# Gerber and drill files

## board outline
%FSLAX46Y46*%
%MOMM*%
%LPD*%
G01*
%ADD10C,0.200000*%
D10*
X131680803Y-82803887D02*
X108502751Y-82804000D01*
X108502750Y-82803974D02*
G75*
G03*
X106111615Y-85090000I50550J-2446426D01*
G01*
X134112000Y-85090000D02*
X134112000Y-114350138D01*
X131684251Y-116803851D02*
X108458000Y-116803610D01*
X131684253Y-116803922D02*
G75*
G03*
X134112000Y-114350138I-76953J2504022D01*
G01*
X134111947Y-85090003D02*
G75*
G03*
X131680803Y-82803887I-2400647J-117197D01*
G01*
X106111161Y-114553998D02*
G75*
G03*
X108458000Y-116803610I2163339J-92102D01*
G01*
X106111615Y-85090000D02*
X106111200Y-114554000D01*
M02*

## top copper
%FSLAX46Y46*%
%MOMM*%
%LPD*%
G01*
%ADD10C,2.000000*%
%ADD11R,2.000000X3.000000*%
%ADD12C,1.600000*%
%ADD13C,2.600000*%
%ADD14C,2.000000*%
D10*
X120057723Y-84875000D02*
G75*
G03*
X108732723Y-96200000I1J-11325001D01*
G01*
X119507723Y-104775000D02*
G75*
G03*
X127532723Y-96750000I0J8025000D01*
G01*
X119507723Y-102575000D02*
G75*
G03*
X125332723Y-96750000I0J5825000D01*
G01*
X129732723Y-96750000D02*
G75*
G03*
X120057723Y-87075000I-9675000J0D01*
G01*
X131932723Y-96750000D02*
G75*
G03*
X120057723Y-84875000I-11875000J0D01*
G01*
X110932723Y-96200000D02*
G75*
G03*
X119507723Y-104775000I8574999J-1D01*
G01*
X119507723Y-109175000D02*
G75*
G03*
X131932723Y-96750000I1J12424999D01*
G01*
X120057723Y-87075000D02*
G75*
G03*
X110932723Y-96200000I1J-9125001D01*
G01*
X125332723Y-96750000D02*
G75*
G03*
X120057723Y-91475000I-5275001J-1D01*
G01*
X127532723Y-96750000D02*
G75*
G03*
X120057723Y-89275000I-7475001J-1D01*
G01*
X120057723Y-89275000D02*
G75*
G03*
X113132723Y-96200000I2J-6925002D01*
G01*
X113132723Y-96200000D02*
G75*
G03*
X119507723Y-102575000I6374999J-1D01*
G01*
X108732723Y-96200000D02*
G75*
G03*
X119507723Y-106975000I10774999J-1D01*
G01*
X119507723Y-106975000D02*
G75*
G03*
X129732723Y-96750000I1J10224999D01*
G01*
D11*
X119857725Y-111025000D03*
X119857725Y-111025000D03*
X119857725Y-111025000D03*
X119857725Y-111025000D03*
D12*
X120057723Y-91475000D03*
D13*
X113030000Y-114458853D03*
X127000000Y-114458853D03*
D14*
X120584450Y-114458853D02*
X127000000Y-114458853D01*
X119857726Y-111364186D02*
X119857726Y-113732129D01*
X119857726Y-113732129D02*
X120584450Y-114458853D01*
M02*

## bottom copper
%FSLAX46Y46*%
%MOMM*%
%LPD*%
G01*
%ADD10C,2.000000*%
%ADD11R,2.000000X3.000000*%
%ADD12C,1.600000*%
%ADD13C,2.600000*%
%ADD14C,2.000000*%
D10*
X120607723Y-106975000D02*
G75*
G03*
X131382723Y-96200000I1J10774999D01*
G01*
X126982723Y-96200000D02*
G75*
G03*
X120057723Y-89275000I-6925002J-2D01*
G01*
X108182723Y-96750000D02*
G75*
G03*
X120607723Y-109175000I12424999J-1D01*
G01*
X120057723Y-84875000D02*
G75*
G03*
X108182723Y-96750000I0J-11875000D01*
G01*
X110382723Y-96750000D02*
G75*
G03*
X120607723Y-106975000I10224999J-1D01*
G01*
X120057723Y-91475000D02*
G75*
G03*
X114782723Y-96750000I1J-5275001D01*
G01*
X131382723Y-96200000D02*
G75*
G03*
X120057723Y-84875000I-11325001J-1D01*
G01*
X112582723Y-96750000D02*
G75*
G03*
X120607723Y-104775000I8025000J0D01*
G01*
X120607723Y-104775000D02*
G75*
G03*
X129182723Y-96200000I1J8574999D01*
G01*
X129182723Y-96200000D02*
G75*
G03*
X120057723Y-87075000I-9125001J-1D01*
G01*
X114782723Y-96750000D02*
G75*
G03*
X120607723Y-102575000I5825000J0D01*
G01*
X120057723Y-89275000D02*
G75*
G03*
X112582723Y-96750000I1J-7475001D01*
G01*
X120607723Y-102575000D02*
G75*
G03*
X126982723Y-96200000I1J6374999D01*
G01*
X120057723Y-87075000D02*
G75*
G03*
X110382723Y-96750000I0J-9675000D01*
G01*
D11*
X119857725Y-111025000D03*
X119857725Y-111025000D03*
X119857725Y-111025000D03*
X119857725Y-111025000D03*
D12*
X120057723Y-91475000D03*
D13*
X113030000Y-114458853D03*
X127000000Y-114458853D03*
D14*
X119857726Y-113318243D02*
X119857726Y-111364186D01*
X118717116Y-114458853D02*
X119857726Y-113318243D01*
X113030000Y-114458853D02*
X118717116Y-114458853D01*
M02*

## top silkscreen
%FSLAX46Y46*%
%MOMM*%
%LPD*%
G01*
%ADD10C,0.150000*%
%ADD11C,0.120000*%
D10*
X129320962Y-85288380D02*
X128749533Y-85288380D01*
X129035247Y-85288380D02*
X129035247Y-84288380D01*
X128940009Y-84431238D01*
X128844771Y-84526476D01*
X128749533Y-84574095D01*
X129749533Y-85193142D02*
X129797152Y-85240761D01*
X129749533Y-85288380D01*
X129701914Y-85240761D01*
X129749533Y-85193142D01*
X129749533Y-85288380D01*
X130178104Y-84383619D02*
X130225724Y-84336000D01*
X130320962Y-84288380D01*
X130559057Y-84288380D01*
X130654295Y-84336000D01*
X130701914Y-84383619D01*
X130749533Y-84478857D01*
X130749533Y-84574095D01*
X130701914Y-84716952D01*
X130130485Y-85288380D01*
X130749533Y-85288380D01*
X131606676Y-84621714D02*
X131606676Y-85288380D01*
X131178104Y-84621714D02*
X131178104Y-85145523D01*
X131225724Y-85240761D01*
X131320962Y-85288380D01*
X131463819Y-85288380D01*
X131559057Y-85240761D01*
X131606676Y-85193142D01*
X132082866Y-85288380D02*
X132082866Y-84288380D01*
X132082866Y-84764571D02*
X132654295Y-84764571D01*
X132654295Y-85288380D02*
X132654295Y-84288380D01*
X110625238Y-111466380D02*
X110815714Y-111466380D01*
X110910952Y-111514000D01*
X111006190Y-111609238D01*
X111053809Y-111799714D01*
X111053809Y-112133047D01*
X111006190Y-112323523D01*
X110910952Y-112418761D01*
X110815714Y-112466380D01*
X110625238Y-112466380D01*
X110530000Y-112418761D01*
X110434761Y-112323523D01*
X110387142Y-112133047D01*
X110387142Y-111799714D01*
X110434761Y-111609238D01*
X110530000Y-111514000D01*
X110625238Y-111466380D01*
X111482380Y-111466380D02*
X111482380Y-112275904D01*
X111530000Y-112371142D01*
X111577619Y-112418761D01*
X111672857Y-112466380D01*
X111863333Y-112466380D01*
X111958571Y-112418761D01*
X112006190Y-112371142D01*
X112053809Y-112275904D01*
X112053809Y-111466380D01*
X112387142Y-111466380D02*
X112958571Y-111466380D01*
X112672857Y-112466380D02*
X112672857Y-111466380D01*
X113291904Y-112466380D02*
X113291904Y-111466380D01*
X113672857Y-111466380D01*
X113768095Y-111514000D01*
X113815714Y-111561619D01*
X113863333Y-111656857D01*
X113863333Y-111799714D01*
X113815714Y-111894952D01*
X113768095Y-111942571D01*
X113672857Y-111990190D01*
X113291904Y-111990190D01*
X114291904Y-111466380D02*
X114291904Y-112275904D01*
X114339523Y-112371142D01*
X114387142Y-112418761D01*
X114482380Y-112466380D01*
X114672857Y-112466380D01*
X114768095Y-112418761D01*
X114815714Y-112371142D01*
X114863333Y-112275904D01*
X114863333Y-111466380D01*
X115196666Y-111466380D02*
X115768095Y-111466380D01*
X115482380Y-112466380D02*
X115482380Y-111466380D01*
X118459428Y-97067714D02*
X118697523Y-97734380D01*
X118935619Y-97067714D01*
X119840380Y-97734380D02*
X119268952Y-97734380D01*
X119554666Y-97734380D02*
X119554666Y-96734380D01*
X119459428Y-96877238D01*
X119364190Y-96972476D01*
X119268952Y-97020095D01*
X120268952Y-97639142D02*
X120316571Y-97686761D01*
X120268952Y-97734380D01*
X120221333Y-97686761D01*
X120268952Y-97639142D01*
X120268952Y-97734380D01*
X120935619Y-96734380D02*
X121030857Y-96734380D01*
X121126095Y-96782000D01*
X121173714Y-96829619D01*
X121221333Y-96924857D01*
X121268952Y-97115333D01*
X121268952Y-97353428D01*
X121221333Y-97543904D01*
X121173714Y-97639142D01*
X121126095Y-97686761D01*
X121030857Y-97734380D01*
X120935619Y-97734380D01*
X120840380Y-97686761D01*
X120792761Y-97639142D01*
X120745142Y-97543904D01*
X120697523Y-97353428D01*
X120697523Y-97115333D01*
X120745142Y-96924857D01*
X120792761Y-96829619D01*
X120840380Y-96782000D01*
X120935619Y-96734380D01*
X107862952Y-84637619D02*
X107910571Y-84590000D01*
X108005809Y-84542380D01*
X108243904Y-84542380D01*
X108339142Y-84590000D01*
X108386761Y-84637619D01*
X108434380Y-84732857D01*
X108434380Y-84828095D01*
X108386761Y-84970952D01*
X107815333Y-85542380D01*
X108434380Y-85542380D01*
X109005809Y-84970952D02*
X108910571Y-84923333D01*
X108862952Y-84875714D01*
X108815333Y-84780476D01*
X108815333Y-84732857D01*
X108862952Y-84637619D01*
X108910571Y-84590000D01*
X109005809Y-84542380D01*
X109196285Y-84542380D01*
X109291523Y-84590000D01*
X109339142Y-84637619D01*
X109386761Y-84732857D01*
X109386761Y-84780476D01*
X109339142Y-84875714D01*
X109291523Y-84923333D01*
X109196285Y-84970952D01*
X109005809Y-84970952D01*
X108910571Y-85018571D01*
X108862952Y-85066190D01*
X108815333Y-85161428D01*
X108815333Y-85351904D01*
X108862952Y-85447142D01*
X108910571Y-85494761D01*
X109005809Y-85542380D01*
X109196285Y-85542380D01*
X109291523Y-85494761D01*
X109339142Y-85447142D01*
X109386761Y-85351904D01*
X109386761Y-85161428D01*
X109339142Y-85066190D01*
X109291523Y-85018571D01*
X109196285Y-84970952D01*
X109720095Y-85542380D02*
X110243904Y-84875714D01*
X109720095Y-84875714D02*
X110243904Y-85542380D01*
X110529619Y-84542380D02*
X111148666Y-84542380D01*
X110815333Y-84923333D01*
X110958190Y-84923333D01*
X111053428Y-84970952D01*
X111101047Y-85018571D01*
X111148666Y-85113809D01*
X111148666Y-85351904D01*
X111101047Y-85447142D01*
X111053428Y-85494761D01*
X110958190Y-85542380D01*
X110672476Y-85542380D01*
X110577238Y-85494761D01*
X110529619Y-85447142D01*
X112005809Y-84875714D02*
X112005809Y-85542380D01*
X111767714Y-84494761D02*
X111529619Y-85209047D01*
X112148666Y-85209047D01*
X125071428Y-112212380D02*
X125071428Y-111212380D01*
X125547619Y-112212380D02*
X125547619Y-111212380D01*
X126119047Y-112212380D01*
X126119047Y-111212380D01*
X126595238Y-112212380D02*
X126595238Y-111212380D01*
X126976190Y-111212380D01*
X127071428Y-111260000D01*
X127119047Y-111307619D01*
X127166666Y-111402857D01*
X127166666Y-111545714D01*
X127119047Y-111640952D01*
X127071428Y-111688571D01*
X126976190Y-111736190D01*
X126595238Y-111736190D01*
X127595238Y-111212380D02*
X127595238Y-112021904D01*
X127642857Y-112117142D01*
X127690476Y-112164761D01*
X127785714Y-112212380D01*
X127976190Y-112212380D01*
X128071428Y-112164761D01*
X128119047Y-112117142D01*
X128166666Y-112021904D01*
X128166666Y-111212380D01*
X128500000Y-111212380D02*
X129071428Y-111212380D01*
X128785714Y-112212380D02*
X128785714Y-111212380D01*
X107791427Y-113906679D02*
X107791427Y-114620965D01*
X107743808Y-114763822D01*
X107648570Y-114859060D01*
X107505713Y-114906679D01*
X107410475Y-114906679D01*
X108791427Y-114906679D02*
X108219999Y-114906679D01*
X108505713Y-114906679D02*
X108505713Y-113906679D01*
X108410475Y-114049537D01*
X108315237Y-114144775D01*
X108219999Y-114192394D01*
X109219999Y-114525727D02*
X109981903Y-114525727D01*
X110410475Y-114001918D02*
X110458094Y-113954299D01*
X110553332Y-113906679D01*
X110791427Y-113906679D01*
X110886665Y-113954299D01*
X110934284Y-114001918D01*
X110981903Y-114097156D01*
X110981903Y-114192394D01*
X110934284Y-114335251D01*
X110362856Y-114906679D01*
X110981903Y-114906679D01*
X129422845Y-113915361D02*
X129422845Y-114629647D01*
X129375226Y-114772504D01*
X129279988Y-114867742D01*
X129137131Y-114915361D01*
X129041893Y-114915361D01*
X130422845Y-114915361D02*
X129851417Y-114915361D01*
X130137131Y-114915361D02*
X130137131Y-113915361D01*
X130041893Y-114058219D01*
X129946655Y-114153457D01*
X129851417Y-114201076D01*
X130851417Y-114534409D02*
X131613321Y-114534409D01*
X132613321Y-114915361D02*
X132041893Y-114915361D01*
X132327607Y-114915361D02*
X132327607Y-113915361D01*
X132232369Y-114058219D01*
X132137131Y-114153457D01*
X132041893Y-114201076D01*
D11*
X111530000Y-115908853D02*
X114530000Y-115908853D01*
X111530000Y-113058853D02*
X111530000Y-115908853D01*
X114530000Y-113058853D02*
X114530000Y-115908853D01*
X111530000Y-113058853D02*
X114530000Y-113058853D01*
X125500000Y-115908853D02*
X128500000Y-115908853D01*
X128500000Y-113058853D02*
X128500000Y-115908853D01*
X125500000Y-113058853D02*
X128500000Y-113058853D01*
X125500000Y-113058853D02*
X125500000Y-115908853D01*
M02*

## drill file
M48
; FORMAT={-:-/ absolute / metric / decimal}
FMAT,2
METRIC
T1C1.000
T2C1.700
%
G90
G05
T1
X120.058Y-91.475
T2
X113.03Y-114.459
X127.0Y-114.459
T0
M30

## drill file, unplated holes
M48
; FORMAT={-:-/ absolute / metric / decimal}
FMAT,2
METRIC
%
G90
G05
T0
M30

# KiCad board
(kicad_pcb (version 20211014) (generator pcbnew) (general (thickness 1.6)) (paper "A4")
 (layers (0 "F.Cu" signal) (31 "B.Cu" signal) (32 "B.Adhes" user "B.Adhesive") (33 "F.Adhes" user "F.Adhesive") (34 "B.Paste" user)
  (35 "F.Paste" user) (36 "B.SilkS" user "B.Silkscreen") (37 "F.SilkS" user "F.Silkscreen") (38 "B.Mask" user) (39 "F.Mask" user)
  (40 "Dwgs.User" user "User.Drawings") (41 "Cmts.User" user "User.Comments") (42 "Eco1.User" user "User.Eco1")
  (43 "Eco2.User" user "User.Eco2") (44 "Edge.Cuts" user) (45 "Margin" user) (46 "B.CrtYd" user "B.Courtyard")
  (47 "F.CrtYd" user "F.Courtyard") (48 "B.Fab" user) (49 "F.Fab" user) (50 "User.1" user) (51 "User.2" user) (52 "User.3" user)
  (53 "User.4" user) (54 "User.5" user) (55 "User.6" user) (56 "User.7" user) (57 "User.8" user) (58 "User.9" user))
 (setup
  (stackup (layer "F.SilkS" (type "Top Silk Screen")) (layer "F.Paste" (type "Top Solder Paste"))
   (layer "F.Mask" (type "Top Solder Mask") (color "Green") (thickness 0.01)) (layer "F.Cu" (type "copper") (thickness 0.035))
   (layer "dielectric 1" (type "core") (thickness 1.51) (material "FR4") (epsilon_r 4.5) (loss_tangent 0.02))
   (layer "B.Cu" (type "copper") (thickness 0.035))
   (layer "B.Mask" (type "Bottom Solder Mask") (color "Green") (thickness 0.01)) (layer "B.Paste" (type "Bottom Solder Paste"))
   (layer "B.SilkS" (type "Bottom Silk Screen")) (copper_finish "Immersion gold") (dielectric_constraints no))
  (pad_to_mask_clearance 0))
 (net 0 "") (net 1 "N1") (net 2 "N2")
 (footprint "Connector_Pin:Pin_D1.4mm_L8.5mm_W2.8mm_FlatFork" (layer "F.Cu") (at 113.03 114.458853)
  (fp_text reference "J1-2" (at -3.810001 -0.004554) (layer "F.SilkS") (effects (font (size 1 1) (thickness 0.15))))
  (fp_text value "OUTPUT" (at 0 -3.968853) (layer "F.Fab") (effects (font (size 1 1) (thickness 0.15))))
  (fp_line (start -1.5 1.45) (end 1.5 1.45) (layer "F.SilkS") (width 0.12))
  (fp_line (start -1.5 -1.4) (end -1.5 1.45) (layer "F.SilkS") (width 0.12))
  (fp_line (start 1.5 -1.4) (end 1.5 1.45) (layer "F.SilkS") (width 0.12))
  (fp_line (start -1.5 -1.4) (end 1.5 -1.4) (layer "F.SilkS") (width 0.12))
  (pad "1" thru_hole circle locked (at 0 0) (size 2.6 2.6) (drill 1.7) (layers *.Cu *.Mask) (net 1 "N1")))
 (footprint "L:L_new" (layer "F.Cu") (at 120.057723 98.2 90) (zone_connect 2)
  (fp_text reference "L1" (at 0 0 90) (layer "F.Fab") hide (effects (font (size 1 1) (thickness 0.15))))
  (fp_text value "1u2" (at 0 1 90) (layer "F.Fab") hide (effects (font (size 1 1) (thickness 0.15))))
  (fp_arc (start 1.45 7.475) (mid -4.224532 5.124532) (end -6.575 -0.55) (layer "F.Cu") (width 2))
  (fp_arc (start -4.375 -0.55) (mid -2.507806 -5.057806) (end 2 -6.925) (layer "F.Cu") (width 2))
  (fp_arc (start 2 -6.925) (mid 6.896714 -4.896714) (end 8.925 0) (layer "F.Cu") (width 2))
  (fp_arc (start 1.45 11.875) (mid -7.335802 8.235802) (end -10.975 -0.55) (layer "F.Cu") (width 2))
  (fp_arc (start 1.45 9.675) (mid -5.780167 6.680167) (end -8.775 -0.55) (layer "F.Cu") (width 2))
  (fp_arc (start -8.775 -0.55) (mid -5.619076 -8.169076) (end 2 -11.325) (layer "F.Cu") (width 2))
  (fp_arc (start 8.925 0) (mid 6.735623 5.285623) (end 1.45 7.475) (layer "F.Cu") (width 2))
  (fp_arc (start 13.325 0) (mid 9.846893 8.396893) (end 1.45 11.875) (layer "F.Cu") (width 2))
  (fp_arc (start 11.125 0) (mid 8.291258 6.841258) (end 1.45 9.675) (layer "F.Cu") (width 2))
  (fp_arc (start 2 -11.325) (mid 10.007984 -8.007984) (end 13.325 0) (layer "F.Cu") (width 2))
  (fp_arc (start 1.45 5.275) (mid -2.668897 3.568897) (end -4.375 -0.55) (layer "F.Cu") (width 2))
  (fp_arc (start 2 -9.125) (mid 8.452349 -6.452349) (end 11.125 0) (layer "F.Cu") (width 2))
  (fp_arc (start -6.575 -0.55) (mid -4.063441 -6.613441) (end 2 -9.125) (layer "F.Cu") (width 2))
  (fp_arc (start 6.725 0) (mid 5.179988 3.729988) (end 1.45 5.275) (layer "F.Cu") (width 2))
  (fp_arc (start -8.775 0.55) (mid -5.780167 -6.680167) (end 1.45 -9.675) (layer "B.Cu") (width 2))
  (fp_arc (start 2 11.325) (mid -5.619076 8.169076) (end -8.775 0.55) (layer "B.Cu") (width 2))
  (fp_arc (start 1.45 -7.475) (mid 6.735623 -5.285623) (end 8.925 0) (layer "B.Cu") (width 2))
  (fp_arc (start 1.45 -9.675) (mid 8.291258 -6.841258) (end 11.125 0) (layer "B.Cu") (width 2))
  (fp_arc (start 13.325 0) (mid 10.007984 8.007984) (end 2 11.325) (layer "B.Cu") (width 2))
  (fp_arc (start 11.125 0) (mid 8.452349 6.452349) (end 2 9.125) (layer "B.Cu") (width 2))
  (fp_arc (start 2 9.125) (mid -4.063441 6.613441) (end -6.575 0.55) (layer "B.Cu") (width 2))
  (fp_arc (start -4.375 0.55) (mid -2.668897 -3.568897) (end 1.45 -5.275) (layer "B.Cu") (width 2))
  (fp_arc (start 8.925 0) (mid 6.896714 4.896714) (end 2 6.925) (layer "B.Cu") (width 2))
  (fp_arc (start -10.975 0.55) (mid -7.335802 -8.235802) (end 1.45 -11.875) (layer "B.Cu") (width 2))
  (fp_arc (start 2 6.925) (mid -2.507806 5.057806) (end -4.375 0.55) (layer "B.Cu") (width 2))
  (fp_arc (start 1.45 -5.275) (mid 5.179988 -3.729988) (end 6.725 0) (layer "B.Cu") (width 2))
  (fp_arc (start 1.45 -11.875) (mid 9.846893 -8.396893) (end 13.325 0) (layer "B.Cu") (width 2))
  (fp_arc (start -6.575 0.55) (mid -4.224532 -5.124532) (end 1.45 -7.475) (layer "B.Cu") (width 2))
  (pad "1" smd rect (at -12.825 -0.199998 90) (size 3 2) (layers *.Mask "F.Cu" "F.Paste") (zone_connect 2))
  (pad "1" smd rect (at -12.825 -0.199998 90) (size 3 2) (layers *.Mask "F.Cu" "F.Paste") (zone_connect 2))
  (pad "1" smd rect (at -12.825 -0.199998 90) (size 3 2) (layers *.Mask "F.Cu" "F.Paste") (zone_connect 2))
  (pad "1" smd rect (at -12.825 -0.199998 90) (size 3 2) (layers *.Mask "F.Cu" "F.Paste") (zone_connect 2))
  (pad "2" smd rect (at -12.825 -0.199998 90) (size 3 2) (layers "B.Cu" "B.Paste" "B.Mask") (zone_connect 2))
  (pad "2" smd rect (at -12.825 -0.199998 90) (size 3 2) (layers "B.Cu" "B.Paste" "B.Mask") (zone_connect 2))
  (pad "2" smd rect (at -12.825 -0.199998 90) (size 3 2) (layers "B.Cu" "B.Paste" "B.Mask") (zone_connect 2))
  (pad "2" smd rect (at -12.825 -0.199998 90) (size 3 2) (layers "B.Cu" "B.Paste" "B.Mask") (zone_connect 2))
  (pad "lc" thru_hole circle locked (at 6.725 0 90) (size 1.6 1.6) (drill 1) (layers *.Cu *.Mask) (zone_connect 2)))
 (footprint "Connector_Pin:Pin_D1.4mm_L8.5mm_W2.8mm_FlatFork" (layer "F.Cu") (at 127 114.458853)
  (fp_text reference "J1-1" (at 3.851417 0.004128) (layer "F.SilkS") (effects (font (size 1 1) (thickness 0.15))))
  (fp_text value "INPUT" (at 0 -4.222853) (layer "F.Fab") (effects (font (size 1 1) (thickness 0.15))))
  (fp_line (start -1.5 1.45) (end 1.5 1.45) (layer "F.SilkS") (width 0.12))
  (fp_line (start 1.5 -1.4) (end 1.5 1.45) (layer "F.SilkS") (width 0.12))
  (fp_line (start -1.5 -1.4) (end 1.5 -1.4) (layer "F.SilkS") (width 0.12))
  (fp_line (start -1.5 -1.4) (end -1.5 1.45) (layer "F.SilkS") (width 0.12))
  (pad "1" thru_hole circle locked (at 0 0) (size 2.6 2.6) (drill 1.7) (layers *.Cu *.Mask) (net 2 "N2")))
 (gr_line (start 131.680803 82.803887) (end 108.502751 82.804) (layer "Edge.Cuts") (width 0.2))
 (gr_arc (start 106.111615 85.09) (mid 106.86236 83.481719) (end 108.502751 82.804) (layer "Edge.Cuts") (width 0.2))
 (gr_line (start 134.112 85.09) (end 134.112 114.350138) (layer "Edge.Cuts") (width 0.2))
 (gr_line (start 131.684251 116.803851) (end 108.458 116.80361) (layer "Edge.Cuts") (width 0.2))
 (gr_arc (start 134.112 114.350138) (mid 133.388153 116.061837) (end 131.684251 116.803851) (layer "Edge.Cuts") (width 0.2))
 (gr_arc (start 131.680803 82.803887) (mid 133.357835 83.456226) (end 134.112 85.09) (layer "Edge.Cuts") (width 0.2))
 (gr_arc (start 108.458 116.80361) (mid 106.77615 116.209221) (end 106.1112 114.554) (layer "Edge.Cuts") (width 0.2))
 (gr_line (start 106.111615 85.09) (end 106.1112 114.554) (layer "Edge.Cuts") (width 0.2))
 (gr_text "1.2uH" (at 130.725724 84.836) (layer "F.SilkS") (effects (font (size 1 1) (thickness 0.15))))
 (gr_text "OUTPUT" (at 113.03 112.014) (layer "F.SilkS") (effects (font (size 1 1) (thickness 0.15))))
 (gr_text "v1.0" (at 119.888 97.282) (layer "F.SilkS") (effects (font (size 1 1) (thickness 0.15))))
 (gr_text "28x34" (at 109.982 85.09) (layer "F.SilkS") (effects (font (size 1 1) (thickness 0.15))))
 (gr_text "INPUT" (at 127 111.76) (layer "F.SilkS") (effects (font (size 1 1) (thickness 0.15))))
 (segment (start 120.58445 114.458853) (end 127 114.458853) (width 2) (layer "F.Cu") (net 2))
 (segment (start 119.857726 111.364186) (end 119.857726 113.732129) (width 2) (layer "F.Cu") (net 2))
 (segment (start 119.857726 113.732129) (end 120.58445 114.458853) (width 2) (layer "F.Cu") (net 2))
 (segment (start 118.717116 114.458853) (end 119.857726 113.318243) (width 2) (layer "B.Cu") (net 1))
 (segment (start 119.857726 113.318243) (end 119.857726 111.364186) (width 2) (layer "B.Cu") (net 1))
 (segment (start 113.03 114.458853) (end 118.717116 114.458853) (width 2) (layer "B.Cu") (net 1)))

